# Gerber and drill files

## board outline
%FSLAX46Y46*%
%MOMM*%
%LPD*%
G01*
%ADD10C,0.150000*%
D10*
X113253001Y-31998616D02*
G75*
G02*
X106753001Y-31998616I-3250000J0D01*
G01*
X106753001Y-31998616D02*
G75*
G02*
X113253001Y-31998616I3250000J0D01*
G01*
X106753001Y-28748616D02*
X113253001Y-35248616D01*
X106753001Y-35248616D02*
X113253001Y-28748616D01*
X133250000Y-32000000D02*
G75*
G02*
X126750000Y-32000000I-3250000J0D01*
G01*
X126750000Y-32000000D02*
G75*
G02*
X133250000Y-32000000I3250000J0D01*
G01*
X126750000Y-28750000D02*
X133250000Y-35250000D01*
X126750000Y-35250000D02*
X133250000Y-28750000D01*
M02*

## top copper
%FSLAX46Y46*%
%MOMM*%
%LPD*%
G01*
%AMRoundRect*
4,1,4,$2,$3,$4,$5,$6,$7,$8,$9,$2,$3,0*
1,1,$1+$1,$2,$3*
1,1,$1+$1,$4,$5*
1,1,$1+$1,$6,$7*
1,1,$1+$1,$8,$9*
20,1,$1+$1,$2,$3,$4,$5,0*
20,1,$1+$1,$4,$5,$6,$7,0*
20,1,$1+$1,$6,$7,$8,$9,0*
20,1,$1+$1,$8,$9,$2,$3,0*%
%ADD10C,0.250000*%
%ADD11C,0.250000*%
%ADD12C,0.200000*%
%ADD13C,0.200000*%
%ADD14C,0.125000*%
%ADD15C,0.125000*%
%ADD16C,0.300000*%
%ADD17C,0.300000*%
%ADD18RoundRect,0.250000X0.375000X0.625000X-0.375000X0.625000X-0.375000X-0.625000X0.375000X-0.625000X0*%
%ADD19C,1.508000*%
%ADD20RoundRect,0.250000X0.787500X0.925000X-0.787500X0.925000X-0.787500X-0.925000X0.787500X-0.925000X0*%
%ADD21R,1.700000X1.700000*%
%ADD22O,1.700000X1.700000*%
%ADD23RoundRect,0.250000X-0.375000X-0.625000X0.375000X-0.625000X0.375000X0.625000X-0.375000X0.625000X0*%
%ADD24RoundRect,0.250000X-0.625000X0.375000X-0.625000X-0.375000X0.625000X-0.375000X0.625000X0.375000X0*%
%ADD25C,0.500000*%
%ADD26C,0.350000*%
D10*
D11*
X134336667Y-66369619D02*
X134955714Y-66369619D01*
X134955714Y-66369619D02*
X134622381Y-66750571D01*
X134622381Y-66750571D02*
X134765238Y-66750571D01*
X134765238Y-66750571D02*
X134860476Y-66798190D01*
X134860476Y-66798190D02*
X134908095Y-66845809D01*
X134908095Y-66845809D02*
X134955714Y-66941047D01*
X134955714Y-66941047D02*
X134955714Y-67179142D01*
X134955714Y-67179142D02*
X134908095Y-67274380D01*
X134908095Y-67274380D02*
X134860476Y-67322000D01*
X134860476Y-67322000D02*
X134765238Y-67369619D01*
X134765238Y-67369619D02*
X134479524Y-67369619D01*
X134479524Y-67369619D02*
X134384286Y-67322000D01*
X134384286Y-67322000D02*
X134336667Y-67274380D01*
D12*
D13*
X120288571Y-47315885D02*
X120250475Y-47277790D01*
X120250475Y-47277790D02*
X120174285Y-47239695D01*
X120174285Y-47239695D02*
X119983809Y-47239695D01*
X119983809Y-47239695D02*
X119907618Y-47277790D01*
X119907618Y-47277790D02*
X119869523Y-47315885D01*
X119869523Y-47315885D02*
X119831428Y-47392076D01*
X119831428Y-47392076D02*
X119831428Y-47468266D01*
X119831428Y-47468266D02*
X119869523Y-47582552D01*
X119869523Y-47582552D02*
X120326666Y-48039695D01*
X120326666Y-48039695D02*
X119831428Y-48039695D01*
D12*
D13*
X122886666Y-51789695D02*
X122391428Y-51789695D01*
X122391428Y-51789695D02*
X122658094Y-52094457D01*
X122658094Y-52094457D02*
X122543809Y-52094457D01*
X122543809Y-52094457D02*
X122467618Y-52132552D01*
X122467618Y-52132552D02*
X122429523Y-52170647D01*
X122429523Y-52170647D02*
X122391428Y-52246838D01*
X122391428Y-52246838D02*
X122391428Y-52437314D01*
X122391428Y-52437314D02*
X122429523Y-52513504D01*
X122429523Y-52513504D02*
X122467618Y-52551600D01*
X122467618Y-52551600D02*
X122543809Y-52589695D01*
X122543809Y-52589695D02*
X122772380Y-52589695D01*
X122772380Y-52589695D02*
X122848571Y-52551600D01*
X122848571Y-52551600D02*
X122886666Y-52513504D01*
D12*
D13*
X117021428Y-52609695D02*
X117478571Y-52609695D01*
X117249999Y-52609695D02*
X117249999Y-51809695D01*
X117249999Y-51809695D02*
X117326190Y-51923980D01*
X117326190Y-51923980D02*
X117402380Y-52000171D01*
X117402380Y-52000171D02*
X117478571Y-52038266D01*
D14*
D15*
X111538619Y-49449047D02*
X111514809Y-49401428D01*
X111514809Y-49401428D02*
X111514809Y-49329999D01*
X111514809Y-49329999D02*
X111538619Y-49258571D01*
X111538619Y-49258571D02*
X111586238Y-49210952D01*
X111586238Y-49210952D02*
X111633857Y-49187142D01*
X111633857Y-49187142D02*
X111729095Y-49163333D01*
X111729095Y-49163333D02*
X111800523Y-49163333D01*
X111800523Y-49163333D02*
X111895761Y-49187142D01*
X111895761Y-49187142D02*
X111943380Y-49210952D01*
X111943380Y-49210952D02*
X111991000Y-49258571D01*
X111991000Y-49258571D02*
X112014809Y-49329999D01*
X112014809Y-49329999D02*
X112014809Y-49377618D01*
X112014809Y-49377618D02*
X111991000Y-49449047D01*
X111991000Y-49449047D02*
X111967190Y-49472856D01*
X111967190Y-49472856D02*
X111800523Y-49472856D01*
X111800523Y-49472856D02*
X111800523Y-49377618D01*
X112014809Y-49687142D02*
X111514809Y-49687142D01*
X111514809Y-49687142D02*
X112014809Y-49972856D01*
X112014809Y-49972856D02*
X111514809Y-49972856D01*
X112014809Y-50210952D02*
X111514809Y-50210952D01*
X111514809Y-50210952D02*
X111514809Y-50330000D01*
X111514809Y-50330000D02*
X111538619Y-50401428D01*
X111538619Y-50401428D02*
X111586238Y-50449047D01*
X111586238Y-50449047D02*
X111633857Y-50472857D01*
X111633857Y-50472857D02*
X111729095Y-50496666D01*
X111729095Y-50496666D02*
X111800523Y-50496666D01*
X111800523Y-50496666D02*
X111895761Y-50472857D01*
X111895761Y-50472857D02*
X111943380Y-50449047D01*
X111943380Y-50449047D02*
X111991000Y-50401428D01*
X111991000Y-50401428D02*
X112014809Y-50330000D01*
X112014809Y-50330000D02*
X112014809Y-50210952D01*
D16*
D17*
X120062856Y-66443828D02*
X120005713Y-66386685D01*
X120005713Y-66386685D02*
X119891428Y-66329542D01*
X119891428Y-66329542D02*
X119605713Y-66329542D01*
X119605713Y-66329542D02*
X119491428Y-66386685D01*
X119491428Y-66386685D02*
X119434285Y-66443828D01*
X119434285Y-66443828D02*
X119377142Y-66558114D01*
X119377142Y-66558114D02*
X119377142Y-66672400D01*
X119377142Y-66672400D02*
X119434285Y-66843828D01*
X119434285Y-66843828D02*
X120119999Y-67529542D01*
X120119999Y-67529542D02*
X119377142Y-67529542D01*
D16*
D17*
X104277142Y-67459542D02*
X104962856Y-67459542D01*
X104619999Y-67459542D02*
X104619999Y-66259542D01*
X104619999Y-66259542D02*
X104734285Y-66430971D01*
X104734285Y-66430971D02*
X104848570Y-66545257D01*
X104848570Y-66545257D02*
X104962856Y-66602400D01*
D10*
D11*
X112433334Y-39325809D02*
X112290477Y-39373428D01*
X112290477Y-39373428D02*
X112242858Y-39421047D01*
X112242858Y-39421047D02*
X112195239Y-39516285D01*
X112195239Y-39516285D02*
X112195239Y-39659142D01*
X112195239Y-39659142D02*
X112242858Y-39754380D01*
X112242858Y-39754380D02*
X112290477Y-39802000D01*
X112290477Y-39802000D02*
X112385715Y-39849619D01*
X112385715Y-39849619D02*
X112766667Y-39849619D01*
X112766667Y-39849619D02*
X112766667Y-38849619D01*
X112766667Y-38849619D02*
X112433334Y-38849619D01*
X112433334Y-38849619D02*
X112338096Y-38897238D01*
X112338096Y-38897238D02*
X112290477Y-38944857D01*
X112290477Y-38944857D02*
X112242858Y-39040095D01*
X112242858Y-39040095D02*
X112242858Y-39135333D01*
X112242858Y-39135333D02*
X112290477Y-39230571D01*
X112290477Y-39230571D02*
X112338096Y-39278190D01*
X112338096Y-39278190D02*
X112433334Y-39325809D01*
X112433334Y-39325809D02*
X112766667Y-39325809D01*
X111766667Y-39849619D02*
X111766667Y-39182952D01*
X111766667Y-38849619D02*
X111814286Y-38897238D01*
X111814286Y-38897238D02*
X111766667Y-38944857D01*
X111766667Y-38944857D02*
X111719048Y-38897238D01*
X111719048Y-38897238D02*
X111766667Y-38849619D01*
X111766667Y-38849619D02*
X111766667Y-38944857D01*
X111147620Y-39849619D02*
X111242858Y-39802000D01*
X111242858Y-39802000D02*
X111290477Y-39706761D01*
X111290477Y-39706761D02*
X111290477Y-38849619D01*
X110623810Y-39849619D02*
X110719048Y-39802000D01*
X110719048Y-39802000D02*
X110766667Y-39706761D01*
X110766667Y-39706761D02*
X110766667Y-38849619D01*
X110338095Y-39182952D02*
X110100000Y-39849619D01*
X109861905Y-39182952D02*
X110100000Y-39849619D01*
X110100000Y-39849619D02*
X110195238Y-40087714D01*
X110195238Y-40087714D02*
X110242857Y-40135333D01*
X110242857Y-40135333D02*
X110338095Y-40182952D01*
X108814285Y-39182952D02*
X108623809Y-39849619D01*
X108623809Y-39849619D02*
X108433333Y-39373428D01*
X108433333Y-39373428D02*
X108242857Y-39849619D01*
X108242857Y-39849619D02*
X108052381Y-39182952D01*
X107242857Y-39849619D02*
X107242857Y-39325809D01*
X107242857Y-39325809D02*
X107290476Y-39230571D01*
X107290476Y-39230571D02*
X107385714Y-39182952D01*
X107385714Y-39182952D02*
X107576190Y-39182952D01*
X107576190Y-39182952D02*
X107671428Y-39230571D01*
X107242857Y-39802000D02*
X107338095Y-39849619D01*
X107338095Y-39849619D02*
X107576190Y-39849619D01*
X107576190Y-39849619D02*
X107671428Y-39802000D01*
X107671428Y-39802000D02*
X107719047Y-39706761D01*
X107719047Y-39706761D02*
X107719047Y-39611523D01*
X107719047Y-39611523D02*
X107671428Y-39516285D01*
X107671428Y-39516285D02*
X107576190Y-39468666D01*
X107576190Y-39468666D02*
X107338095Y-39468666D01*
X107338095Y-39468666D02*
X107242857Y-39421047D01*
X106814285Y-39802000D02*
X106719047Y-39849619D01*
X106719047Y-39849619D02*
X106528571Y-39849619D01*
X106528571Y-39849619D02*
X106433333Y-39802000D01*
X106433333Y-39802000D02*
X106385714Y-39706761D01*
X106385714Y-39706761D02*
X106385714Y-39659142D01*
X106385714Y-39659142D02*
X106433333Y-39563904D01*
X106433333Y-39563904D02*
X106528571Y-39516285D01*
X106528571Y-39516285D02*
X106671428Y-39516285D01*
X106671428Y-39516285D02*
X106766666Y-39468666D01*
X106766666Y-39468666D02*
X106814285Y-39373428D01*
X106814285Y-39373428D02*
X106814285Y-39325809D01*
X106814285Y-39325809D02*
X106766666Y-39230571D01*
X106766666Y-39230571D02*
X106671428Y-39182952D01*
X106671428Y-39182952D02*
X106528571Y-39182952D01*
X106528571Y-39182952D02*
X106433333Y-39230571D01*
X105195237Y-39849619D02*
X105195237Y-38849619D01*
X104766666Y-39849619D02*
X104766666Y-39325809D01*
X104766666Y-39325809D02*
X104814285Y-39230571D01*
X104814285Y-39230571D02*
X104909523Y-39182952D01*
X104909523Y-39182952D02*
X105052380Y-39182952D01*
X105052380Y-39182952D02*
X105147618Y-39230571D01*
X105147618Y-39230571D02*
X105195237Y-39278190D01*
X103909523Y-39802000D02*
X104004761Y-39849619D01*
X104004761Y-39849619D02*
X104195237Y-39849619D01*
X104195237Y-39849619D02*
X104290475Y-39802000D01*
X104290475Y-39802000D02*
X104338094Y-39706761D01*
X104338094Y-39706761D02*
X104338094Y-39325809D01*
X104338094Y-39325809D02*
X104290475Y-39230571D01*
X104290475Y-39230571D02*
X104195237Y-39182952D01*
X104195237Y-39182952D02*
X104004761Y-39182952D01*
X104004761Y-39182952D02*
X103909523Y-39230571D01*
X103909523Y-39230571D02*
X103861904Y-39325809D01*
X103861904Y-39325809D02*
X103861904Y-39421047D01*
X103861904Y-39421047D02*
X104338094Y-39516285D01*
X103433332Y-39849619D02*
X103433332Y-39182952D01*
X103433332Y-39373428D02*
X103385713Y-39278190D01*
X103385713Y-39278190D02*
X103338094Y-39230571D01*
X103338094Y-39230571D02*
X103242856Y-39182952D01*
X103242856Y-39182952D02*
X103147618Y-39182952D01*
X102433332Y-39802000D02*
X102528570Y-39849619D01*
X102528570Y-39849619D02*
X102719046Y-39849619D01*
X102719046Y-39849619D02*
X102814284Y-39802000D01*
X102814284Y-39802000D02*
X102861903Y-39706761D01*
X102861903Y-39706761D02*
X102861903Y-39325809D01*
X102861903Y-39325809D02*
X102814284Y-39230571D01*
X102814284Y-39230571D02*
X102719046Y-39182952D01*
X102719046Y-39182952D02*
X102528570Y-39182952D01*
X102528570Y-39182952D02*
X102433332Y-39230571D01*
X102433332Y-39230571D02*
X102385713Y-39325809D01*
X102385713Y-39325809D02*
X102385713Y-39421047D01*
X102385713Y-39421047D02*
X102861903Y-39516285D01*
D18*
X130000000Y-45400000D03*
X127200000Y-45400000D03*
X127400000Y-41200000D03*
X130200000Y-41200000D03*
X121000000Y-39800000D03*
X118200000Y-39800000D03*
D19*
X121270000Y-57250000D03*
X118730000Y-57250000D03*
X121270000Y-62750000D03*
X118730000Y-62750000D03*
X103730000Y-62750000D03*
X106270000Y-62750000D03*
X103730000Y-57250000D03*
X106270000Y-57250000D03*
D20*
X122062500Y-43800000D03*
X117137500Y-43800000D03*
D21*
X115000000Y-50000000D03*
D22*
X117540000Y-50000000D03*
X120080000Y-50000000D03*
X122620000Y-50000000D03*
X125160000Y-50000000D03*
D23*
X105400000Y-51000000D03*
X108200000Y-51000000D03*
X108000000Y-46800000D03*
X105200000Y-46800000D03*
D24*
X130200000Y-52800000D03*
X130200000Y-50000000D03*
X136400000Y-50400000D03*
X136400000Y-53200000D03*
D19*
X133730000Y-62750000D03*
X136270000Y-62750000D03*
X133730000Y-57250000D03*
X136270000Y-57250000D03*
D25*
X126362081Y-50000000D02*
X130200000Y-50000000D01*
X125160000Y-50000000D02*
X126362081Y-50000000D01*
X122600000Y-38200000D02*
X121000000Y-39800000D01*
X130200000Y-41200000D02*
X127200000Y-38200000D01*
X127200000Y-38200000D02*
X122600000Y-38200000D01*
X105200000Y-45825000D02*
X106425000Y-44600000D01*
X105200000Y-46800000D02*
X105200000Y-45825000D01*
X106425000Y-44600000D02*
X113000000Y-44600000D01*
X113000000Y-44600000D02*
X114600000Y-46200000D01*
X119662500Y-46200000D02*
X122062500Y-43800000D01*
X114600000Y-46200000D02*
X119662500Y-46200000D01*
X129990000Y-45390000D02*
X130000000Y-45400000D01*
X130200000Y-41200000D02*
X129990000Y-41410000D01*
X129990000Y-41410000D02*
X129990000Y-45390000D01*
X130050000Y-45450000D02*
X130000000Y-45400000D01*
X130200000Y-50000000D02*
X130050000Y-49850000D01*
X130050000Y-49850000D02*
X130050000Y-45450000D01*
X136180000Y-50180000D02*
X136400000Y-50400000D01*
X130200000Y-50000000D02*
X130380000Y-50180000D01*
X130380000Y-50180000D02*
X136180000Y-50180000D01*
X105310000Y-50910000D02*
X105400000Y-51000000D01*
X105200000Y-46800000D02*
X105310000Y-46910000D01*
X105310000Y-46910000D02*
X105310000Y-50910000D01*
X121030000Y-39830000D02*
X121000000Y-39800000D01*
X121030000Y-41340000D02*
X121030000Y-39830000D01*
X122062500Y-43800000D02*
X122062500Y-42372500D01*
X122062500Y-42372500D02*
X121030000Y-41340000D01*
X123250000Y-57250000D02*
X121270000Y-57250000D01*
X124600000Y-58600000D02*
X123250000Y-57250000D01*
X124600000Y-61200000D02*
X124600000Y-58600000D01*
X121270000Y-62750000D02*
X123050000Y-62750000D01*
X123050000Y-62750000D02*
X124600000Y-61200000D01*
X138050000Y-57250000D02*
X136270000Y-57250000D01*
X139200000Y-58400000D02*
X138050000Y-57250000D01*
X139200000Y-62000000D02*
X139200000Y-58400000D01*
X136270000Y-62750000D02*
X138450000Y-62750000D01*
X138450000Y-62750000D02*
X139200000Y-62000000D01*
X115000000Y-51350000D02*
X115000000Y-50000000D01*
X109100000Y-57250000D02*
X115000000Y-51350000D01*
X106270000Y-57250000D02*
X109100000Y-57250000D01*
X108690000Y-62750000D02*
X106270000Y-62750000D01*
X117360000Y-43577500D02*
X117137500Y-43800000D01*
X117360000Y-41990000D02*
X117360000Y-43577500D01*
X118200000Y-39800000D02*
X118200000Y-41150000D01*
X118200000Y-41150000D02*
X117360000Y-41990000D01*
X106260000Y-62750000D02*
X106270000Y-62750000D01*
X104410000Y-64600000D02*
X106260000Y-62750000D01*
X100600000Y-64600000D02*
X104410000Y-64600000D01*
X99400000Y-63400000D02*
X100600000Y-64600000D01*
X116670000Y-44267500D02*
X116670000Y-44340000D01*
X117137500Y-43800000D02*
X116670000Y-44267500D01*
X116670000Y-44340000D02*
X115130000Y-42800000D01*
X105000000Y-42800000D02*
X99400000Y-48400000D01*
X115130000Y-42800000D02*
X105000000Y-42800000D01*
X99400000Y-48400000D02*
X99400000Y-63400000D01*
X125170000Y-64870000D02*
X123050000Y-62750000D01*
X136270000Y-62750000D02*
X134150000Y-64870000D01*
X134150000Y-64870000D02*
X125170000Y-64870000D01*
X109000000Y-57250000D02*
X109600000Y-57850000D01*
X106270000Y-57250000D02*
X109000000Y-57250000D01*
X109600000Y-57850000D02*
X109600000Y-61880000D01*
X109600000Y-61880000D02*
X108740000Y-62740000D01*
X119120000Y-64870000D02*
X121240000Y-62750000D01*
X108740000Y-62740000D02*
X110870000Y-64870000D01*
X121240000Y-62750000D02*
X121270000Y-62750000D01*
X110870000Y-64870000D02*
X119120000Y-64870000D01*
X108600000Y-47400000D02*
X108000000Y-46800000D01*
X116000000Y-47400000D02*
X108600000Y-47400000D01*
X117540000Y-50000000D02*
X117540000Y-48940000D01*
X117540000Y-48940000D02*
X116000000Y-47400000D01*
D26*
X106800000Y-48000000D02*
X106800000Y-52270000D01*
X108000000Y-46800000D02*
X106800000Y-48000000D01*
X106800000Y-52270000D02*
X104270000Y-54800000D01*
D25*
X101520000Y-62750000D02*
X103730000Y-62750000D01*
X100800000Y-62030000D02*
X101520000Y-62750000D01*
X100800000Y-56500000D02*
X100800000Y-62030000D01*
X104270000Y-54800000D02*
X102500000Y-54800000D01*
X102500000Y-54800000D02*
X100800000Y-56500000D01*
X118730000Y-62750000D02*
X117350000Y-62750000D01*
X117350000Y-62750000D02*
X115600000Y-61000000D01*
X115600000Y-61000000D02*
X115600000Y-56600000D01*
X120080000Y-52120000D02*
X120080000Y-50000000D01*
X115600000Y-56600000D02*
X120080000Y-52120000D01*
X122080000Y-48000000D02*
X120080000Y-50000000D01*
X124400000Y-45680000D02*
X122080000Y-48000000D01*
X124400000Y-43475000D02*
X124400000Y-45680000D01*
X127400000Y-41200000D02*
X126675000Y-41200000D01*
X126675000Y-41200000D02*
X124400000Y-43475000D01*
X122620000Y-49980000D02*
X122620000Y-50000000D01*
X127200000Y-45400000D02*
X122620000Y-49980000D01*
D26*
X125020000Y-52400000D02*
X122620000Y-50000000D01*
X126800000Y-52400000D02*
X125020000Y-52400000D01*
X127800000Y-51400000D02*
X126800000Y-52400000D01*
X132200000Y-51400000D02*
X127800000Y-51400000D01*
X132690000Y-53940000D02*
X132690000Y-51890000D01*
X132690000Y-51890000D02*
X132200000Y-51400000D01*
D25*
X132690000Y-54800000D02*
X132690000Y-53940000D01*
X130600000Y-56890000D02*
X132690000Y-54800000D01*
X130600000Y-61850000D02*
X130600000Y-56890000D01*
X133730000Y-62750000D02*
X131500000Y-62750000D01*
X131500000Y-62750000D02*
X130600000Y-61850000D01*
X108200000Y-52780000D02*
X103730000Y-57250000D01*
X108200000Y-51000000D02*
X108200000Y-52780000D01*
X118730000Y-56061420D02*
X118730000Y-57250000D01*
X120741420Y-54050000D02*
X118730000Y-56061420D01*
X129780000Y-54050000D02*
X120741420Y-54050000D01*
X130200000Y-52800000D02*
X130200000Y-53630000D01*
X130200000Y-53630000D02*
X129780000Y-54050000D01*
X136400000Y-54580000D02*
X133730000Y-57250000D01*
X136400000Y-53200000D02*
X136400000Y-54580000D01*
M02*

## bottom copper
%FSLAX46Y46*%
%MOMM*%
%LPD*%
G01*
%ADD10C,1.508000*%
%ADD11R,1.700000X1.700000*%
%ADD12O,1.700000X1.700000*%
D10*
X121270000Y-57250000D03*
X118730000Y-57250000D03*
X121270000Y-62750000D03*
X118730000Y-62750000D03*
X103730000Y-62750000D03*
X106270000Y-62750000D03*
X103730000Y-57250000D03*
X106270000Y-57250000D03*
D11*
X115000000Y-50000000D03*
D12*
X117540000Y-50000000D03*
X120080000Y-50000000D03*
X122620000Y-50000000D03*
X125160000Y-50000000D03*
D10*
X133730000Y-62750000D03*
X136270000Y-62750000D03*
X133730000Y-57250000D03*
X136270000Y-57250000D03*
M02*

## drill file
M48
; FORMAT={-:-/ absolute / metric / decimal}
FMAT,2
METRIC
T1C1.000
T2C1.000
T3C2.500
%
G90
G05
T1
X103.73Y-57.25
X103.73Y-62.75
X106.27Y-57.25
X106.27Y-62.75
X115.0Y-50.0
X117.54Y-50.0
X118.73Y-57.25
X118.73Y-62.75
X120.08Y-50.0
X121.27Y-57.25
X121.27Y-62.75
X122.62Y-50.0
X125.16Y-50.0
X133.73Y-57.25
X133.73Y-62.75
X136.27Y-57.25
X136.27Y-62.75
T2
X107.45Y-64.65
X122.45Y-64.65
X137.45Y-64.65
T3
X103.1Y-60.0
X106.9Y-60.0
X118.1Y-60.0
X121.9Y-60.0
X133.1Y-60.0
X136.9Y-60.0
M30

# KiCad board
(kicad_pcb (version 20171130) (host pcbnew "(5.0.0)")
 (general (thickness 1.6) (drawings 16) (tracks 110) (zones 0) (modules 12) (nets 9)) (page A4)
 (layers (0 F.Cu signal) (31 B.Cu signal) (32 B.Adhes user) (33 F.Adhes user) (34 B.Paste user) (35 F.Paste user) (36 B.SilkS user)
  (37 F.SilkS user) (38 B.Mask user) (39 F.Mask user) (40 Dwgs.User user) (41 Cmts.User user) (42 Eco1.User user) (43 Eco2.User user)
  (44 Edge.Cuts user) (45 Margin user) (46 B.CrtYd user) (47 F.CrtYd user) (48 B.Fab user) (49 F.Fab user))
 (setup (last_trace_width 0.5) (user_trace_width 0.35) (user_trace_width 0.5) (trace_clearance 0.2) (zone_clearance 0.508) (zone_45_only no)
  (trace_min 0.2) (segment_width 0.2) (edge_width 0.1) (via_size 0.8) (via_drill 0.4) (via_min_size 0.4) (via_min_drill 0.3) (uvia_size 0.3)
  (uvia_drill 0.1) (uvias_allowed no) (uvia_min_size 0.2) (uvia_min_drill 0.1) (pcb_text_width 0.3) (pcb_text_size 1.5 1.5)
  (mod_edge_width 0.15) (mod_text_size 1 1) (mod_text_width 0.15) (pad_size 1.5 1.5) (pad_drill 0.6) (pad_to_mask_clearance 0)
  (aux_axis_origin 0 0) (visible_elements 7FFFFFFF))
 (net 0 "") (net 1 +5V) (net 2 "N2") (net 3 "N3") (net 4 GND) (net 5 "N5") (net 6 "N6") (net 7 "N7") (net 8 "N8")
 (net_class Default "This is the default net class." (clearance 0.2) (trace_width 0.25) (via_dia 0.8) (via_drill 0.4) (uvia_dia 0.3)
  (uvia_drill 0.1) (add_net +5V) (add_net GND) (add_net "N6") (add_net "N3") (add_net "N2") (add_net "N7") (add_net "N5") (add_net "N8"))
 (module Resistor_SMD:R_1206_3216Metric (layer F.Cu) (at 128.6 45.4 180)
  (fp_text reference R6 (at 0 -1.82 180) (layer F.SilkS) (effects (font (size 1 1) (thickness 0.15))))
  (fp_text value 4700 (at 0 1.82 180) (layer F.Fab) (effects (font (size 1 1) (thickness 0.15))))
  (pad 1 smd roundrect (at -1.4 0 180) (size 1.25 1.75) (layers F.Cu F.Paste F.Mask) (roundrect_rratio 0.2) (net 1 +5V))
  (pad 2 smd roundrect (at 1.4 0 180) (size 1.25 1.75) (layers F.Cu F.Paste F.Mask) (roundrect_rratio 0.2) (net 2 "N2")))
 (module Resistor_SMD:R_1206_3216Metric (layer F.Cu) (at 128.8 41.2 180)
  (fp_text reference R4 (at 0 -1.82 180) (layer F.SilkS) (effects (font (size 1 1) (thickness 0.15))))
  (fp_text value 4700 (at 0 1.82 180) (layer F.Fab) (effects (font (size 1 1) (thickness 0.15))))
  (pad 2 smd roundrect (at 1.4 0 180) (size 1.25 1.75) (layers F.Cu F.Paste F.Mask) (roundrect_rratio 0.2) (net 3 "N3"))
  (pad 1 smd roundrect (at -1.4 0 180) (size 1.25 1.75) (layers F.Cu F.Paste F.Mask) (roundrect_rratio 0.2) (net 1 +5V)))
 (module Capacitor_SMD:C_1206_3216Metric (layer F.Cu) (at 119.6 39.8 180)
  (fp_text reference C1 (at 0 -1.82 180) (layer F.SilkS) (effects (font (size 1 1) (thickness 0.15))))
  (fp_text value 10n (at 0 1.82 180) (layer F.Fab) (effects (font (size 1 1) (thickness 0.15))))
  (pad 1 smd roundrect (at -1.4 0 180) (size 1.25 1.75) (layers F.Cu F.Paste F.Mask) (roundrect_rratio 0.2) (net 1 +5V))
  (pad 2 smd roundrect (at 1.4 0 180) (size 1.25 1.75) (layers F.Cu F.Paste F.Mask) (roundrect_rratio 0.2) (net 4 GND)))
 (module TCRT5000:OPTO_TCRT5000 (layer F.Cu) (at 120 60 90)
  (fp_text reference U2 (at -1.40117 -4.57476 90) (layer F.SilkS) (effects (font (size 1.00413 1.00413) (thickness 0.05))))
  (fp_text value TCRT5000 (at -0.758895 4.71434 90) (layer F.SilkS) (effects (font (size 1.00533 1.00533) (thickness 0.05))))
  (pad Hole np_thru_hole circle (at 0 -1.9 90) (size 2.5 2.5) (drill 2.5) (layers *.Cu *.Mask F.SilkS))
  (pad Hole np_thru_hole circle (at 0 1.9 90) (size 2.5 2.5) (drill 2.5) (layers *.Cu *.Mask F.SilkS))
  (pad Hole np_thru_hole circle (at -4.65 2.45 90) (size 1 1) (drill 1) (layers *.Cu *.Mask F.SilkS))
  (pad CATH thru_hole circle (at 2.75 1.27 90) (size 1.508 1.508) (drill 1) (layers *.Cu *.Mask) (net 4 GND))
  (pad A thru_hole circle (at 2.75 -1.27 90) (size 1.508 1.508) (drill 1) (layers *.Cu *.Mask) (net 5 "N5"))
  (pad E thru_hole circle (at -2.75 1.27 90) (size 1.508 1.508) (drill 1) (layers *.Cu *.Mask) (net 4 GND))
  (pad COLL thru_hole circle (at -2.75 -1.27 90) (size 1.508 1.508) (drill 1) (layers *.Cu *.Mask) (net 3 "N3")))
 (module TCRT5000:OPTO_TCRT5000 (layer F.Cu) (at 105 60 90)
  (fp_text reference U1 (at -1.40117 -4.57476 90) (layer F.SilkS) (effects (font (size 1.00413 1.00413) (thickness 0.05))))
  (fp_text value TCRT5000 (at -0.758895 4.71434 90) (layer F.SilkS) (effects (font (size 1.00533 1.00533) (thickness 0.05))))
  (pad COLL thru_hole circle (at -2.75 -1.27 90) (size 1.508 1.508) (drill 1) (layers *.Cu *.Mask) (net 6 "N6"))
  (pad E thru_hole circle (at -2.75 1.27 90) (size 1.508 1.508) (drill 1) (layers *.Cu *.Mask) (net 4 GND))
  (pad A thru_hole circle (at 2.75 -1.27 90) (size 1.508 1.508) (drill 1) (layers *.Cu *.Mask) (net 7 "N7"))
  (pad CATH thru_hole circle (at 2.75 1.27 90) (size 1.508 1.508) (drill 1) (layers *.Cu *.Mask) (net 4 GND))
  (pad Hole np_thru_hole circle (at -4.65 2.45 90) (size 1 1) (drill 1) (layers *.Cu *.Mask F.SilkS))
  (pad Hole np_thru_hole circle (at 0 1.9 90) (size 2.5 2.5) (drill 2.5) (layers *.Cu *.Mask F.SilkS))
  (pad Hole np_thru_hole circle (at 0 -1.9 90) (size 2.5 2.5) (drill 2.5) (layers *.Cu *.Mask F.SilkS)))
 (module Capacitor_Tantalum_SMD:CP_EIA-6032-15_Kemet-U (layer F.Cu) (at 119.6 43.8 180)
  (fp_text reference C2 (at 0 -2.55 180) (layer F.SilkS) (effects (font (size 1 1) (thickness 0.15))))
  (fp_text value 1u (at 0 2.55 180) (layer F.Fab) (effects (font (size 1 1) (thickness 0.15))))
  (pad 1 smd roundrect (at -2.4625 0 180) (size 2.075 2.35) (layers F.Cu F.Paste F.Mask) (roundrect_rratio 0.120482) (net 1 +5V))
  (pad 2 smd roundrect (at 2.4625 0 180) (size 2.075 2.35) (layers F.Cu F.Paste F.Mask) (roundrect_rratio 0.120482) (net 4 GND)))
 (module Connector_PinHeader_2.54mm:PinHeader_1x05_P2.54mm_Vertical (layer F.Cu) (at 115 50 90)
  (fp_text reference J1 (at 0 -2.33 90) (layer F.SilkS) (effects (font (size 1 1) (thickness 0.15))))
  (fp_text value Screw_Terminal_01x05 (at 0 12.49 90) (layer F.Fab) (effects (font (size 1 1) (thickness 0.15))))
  (pad 1 thru_hole rect (at 0 0 90) (size 1.7 1.7) (drill 1) (layers *.Cu *.Mask) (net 4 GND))
  (pad 2 thru_hole oval (at 0 2.54 90) (size 1.7 1.7) (drill 1) (layers *.Cu *.Mask) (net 6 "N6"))
  (pad 3 thru_hole oval (at 0 5.08 90) (size 1.7 1.7) (drill 1) (layers *.Cu *.Mask) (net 3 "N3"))
  (pad 4 thru_hole oval (at 0 7.62 90) (size 1.7 1.7) (drill 1) (layers *.Cu *.Mask) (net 2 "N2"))
  (pad 5 thru_hole oval (at 0 10.16 90) (size 1.7 1.7) (drill 1) (layers *.Cu *.Mask) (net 1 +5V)))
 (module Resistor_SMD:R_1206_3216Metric (layer F.Cu) (at 106.8 51)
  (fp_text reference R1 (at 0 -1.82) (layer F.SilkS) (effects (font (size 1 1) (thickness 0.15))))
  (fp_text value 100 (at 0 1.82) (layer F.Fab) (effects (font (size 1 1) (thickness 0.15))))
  (pad 1 smd roundrect (at -1.4 0) (size 1.25 1.75) (layers F.Cu F.Paste F.Mask) (roundrect_rratio 0.2) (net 1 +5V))
  (pad 2 smd roundrect (at 1.4 0) (size 1.25 1.75) (layers F.Cu F.Paste F.Mask) (roundrect_rratio 0.2) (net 7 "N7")))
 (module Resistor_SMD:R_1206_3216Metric (layer F.Cu) (at 106.6 46.8)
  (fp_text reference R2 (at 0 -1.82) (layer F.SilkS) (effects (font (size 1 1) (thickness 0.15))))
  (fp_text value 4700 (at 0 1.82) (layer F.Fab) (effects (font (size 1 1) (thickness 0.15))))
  (pad 2 smd roundrect (at 1.4 0) (size 1.25 1.75) (layers F.Cu F.Paste F.Mask) (roundrect_rratio 0.2) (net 6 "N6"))
  (pad 1 smd roundrect (at -1.4 0) (size 1.25 1.75) (layers F.Cu F.Paste F.Mask) (roundrect_rratio 0.2) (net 1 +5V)))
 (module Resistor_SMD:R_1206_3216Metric (layer F.Cu) (at 130.2 51.4 270)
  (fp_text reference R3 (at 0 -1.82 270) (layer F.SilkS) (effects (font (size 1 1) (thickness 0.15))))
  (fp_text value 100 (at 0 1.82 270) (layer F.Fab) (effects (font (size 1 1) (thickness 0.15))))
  (pad 2 smd roundrect (at 1.4 0 270) (size 1.25 1.75) (layers F.Cu F.Paste F.Mask) (roundrect_rratio 0.2) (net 5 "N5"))
  (pad 1 smd roundrect (at -1.4 0 270) (size 1.25 1.75) (layers F.Cu F.Paste F.Mask) (roundrect_rratio 0.2) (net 1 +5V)))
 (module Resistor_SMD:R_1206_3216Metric (layer F.Cu) (at 136.4 51.8 270)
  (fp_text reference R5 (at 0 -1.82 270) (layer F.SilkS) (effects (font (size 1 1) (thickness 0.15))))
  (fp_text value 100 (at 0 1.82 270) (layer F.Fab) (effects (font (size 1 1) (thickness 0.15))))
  (pad 1 smd roundrect (at -1.4 0 270) (size 1.25 1.75) (layers F.Cu F.Paste F.Mask) (roundrect_rratio 0.2) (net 1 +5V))
  (pad 2 smd roundrect (at 1.4 0 270) (size 1.25 1.75) (layers F.Cu F.Paste F.Mask) (roundrect_rratio 0.2) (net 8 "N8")))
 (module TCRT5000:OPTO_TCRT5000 (layer F.Cu) (at 135 60 90)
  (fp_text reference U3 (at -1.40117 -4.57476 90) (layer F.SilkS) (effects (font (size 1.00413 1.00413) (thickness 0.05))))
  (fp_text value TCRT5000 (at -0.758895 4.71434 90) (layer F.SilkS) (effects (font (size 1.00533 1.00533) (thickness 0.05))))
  (pad COLL thru_hole circle (at -2.75 -1.27 90) (size 1.508 1.508) (drill 1) (layers *.Cu *.Mask) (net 2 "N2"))
  (pad E thru_hole circle (at -2.75 1.27 90) (size 1.508 1.508) (drill 1) (layers *.Cu *.Mask) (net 4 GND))
  (pad A thru_hole circle (at 2.75 -1.27 90) (size 1.508 1.508) (drill 1) (layers *.Cu *.Mask) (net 8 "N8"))
  (pad CATH thru_hole circle (at 2.75 1.27 90) (size 1.508 1.508) (drill 1) (layers *.Cu *.Mask) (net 4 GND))
  (pad Hole np_thru_hole circle (at -4.65 2.45 90) (size 1 1) (drill 1) (layers *.Cu *.Mask F.SilkS))
  (pad Hole np_thru_hole circle (at 0 1.9 90) (size 2.5 2.5) (drill 2.5) (layers *.Cu *.Mask F.SilkS))
  (pad Hole np_thru_hole circle (at 0 -1.9 90) (size 2.5 2.5) (drill 2.5) (layers *.Cu *.Mask F.SilkS)))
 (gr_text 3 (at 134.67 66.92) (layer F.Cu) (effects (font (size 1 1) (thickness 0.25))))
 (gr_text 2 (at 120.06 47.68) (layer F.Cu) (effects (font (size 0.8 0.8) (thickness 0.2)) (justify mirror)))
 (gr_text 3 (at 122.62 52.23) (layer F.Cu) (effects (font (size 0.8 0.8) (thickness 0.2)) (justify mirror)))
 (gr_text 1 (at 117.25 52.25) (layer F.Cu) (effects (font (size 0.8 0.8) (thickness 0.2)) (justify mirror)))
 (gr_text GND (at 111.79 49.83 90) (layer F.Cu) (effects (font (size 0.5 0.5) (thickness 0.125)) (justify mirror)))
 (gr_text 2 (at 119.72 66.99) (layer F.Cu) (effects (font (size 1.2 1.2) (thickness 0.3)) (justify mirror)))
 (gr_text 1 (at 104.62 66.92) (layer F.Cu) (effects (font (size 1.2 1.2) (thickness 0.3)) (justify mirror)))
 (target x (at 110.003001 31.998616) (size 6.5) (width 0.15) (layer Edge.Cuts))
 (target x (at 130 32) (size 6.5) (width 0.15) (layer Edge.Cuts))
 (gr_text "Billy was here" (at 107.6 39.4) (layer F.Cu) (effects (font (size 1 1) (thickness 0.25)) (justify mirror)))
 (segment (start 126.362081 50) (end 130.2 50) (width 0.5) (layer F.Cu) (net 1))
 (segment (start 125.16 50) (end 126.362081 50) (width 0.5) (layer F.Cu) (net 1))
 (segment (start 122.6 38.2) (end 121 39.8) (width 0.5) (layer F.Cu) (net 1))
 (segment (start 130.2 41.2) (end 127.2 38.2) (width 0.5) (layer F.Cu) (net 1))
 (segment (start 127.2 38.2) (end 122.6 38.2) (width 0.5) (layer F.Cu) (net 1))
 (segment (start 105.2 45.825) (end 106.425 44.6) (width 0.5) (layer F.Cu) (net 1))
 (segment (start 105.2 46.8) (end 105.2 45.825) (width 0.5) (layer F.Cu) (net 1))
 (segment (start 106.425 44.6) (end 113 44.6) (width 0.5) (layer F.Cu) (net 1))
 (segment (start 113 44.6) (end 114.6 46.2) (width 0.5) (layer F.Cu) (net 1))
 (segment (start 119.6625 46.2) (end 122.0625 43.8) (width 0.5) (layer F.Cu) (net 1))
 (segment (start 114.6 46.2) (end 119.6625 46.2) (width 0.5) (layer F.Cu) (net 1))
 (segment (start 129.99 45.39) (end 130 45.4) (width 0.5) (layer F.Cu) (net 1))
 (segment (start 130.2 41.2) (end 129.99 41.41) (width 0.5) (layer F.Cu) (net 1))
 (segment (start 129.99 41.41) (end 129.99 45.39) (width 0.5) (layer F.Cu) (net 1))
 (segment (start 130.05 45.45) (end 130 45.4) (width 0.5) (layer F.Cu) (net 1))
 (segment (start 130.2 50) (end 130.05 49.85) (width 0.5) (layer F.Cu) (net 1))
 (segment (start 130.05 49.85) (end 130.05 45.45) (width 0.5) (layer F.Cu) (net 1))
 (segment (start 136.18 50.18) (end 136.4 50.4) (width 0.5) (layer F.Cu) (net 1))
 (segment (start 130.2 50) (end 130.38 50.18) (width 0.5) (layer F.Cu) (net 1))
 (segment (start 130.38 50.18) (end 136.18 50.18) (width 0.5) (layer F.Cu) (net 1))
 (segment (start 105.31 50.91) (end 105.4 51) (width 0.5) (layer F.Cu) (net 1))
 (segment (start 105.2 46.8) (end 105.31 46.91) (width 0.5) (layer F.Cu) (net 1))
 (segment (start 105.31 46.91) (end 105.31 50.91) (width 0.5) (layer F.Cu) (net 1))
 (segment (start 121.03 39.83) (end 121 39.8) (width 0.5) (layer F.Cu) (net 1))
 (segment (start 121.03 41.34) (end 121.03 39.83) (width 0.5) (layer F.Cu) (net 1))
 (segment (start 122.0625 43.8) (end 122.0625 42.3725) (width 0.5) (layer F.Cu) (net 1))
 (segment (start 122.0625 42.3725) (end 121.03 41.34) (width 0.5) (layer F.Cu) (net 1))
 (segment (start 123.25 57.25) (end 121.27 57.25) (width 0.5) (layer F.Cu) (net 4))
 (segment (start 124.6 58.6) (end 123.25 57.25) (width 0.5) (layer F.Cu) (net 4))
 (segment (start 124.6 61.2) (end 124.6 58.6) (width 0.5) (layer F.Cu) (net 4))
 (segment (start 121.27 62.75) (end 123.05 62.75) (width 0.5) (layer F.Cu) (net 4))
 (segment (start 123.05 62.75) (end 124.6 61.2) (width 0.5) (layer F.Cu) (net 4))
 (segment (start 138.05 57.25) (end 136.27 57.25) (width 0.5) (layer F.Cu) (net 4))
 (segment (start 139.2 58.4) (end 138.05 57.25) (width 0.5) (layer F.Cu) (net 4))
 (segment (start 139.2 62) (end 139.2 58.4) (width 0.5) (layer F.Cu) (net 4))
 (segment (start 136.27 62.75) (end 138.45 62.75) (width 0.5) (layer F.Cu) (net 4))
 (segment (start 138.45 62.75) (end 139.2 62) (width 0.5) (layer F.Cu) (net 4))
 (segment (start 115 51.35) (end 115 50) (width 0.5) (layer F.Cu) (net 4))
 (segment (start 109.1 57.25) (end 115 51.35) (width 0.5) (layer F.Cu) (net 4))
 (segment (start 106.27 57.25) (end 109.1 57.25) (width 0.5) (layer F.Cu) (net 4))
 (segment (start 108.69 62.75) (end 106.27 62.75) (width 0.5) (layer F.Cu) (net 4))
 (segment (start 117.36 43.5775) (end 117.1375 43.8) (width 0.5) (layer F.Cu) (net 4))
 (segment (start 117.36 41.99) (end 117.36 43.5775) (width 0.5) (layer F.Cu) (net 4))
 (segment (start 118.2 39.8) (end 118.2 41.15) (width 0.5) (layer F.Cu) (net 4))
 (segment (start 118.2 41.15) (end 117.36 41.99) (width 0.5) (layer F.Cu) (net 4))
 (segment (start 106.26 62.75) (end 106.27 62.75) (width 0.5) (layer F.Cu) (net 4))
 (segment (start 104.41 64.6) (end 106.26 62.75) (width 0.5) (layer F.Cu) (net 4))
 (segment (start 100.6 64.6) (end 104.41 64.6) (width 0.5) (layer F.Cu) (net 4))
 (segment (start 99.4 63.4) (end 100.6 64.6) (width 0.5) (layer F.Cu) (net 4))
 (segment (start 116.67 44.2675) (end 116.67 44.34) (width 0.5) (layer F.Cu) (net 4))
 (segment (start 117.1375 43.8) (end 116.67 44.2675) (width 0.5) (layer F.Cu) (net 4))
 (segment (start 116.67 44.34) (end 115.13 42.8) (width 0.5) (layer F.Cu) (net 4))
 (segment (start 105 42.8) (end 99.4 48.4) (width 0.5) (layer F.Cu) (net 4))
 (segment (start 115.13 42.8) (end 105 42.8) (width 0.5) (layer F.Cu) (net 4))
 (segment (start 99.4 48.4) (end 99.4 63.4) (width 0.5) (layer F.Cu) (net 4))
 (segment (start 125.17 64.87) (end 123.05 62.75) (width 0.5) (layer F.Cu) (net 4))
 (segment (start 136.27 62.75) (end 134.15 64.87) (width 0.5) (layer F.Cu) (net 4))
 (segment (start 134.15 64.87) (end 125.17 64.87) (width 0.5) (layer F.Cu) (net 4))
 (segment (start 109 57.25) (end 109.6 57.85) (width 0.5) (layer F.Cu) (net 4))
 (segment (start 106.27 57.25) (end 109 57.25) (width 0.5) (layer F.Cu) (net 4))
 (segment (start 109.6 57.85) (end 109.6 61.88) (width 0.5) (layer F.Cu) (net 4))
 (segment (start 109.6 61.88) (end 108.74 62.74) (width 0.5) (layer F.Cu) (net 4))
 (segment (start 119.12 64.87) (end 121.24 62.75) (width 0.5) (layer F.Cu) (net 4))
 (segment (start 108.74 62.74) (end 110.87 64.87) (width 0.5) (layer F.Cu) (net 4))
 (segment (start 121.24 62.75) (end 121.27 62.75) (width 0.5) (layer F.Cu) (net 4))
 (segment (start 110.87 64.87) (end 119.12 64.87) (width 0.5) (layer F.Cu) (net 4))
 (segment (start 108.6 47.4) (end 108 46.8) (width 0.5) (layer F.Cu) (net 6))
 (segment (start 116 47.4) (end 108.6 47.4) (width 0.5) (layer F.Cu) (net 6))
 (segment (start 117.54 50) (end 117.54 48.94) (width 0.5) (layer F.Cu) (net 6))
 (segment (start 117.54 48.94) (end 116 47.4) (width 0.5) (layer F.Cu) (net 6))
 (segment (start 106.8 48) (end 106.8 52.27) (width 0.35) (layer F.Cu) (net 6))
 (segment (start 108 46.8) (end 106.8 48) (width 0.35) (layer F.Cu) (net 6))
 (segment (start 106.8 52.27) (end 104.27 54.8) (width 0.35) (layer F.Cu) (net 6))
 (segment (start 101.52 62.75) (end 103.73 62.75) (width 0.5) (layer F.Cu) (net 6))
 (segment (start 100.8 62.03) (end 101.52 62.75) (width 0.5) (layer F.Cu) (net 6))
 (segment (start 100.8 56.5) (end 100.8 62.03) (width 0.5) (layer F.Cu) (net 6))
 (segment (start 104.27 54.8) (end 102.5 54.8) (width 0.5) (layer F.Cu) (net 6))
 (segment (start 102.5 54.8) (end 100.8 56.5) (width 0.5) (layer F.Cu) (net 6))
 (segment (start 118.73 62.75) (end 117.35 62.75) (width 0.5) (layer F.Cu) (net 3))
 (segment (start 117.35 62.75) (end 115.6 61) (width 0.5) (layer F.Cu) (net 3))
 (segment (start 115.6 61) (end 115.6 56.6) (width 0.5) (layer F.Cu) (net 3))
 (segment (start 120.08 52.12) (end 120.08 50) (width 0.5) (layer F.Cu) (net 3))
 (segment (start 115.6 56.6) (end 120.08 52.12) (width 0.5) (layer F.Cu) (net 3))
 (segment (start 122.08 48) (end 120.08 50) (width 0.5) (layer F.Cu) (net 3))
 (segment (start 124.4 45.68) (end 122.08 48) (width 0.5) (layer F.Cu) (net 3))
 (segment (start 124.4 43.475) (end 124.4 45.68) (width 0.5) (layer F.Cu) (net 3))
 (segment (start 127.4 41.2) (end 126.675 41.2) (width 0.5) (layer F.Cu) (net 3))
 (segment (start 126.675 41.2) (end 124.4 43.475) (width 0.5) (layer F.Cu) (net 3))
 (segment (start 122.62 49.98) (end 122.62 50) (width 0.5) (layer F.Cu) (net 2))
 (segment (start 127.2 45.4) (end 122.62 49.98) (width 0.5) (layer F.Cu) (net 2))
 (segment (start 125.02 52.4) (end 122.62 50) (width 0.35) (layer F.Cu) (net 2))
 (segment (start 126.8 52.4) (end 125.02 52.4) (width 0.35) (layer F.Cu) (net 2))
 (segment (start 127.8 51.4) (end 126.8 52.4) (width 0.35) (layer F.Cu) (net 2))
 (segment (start 132.2 51.4) (end 127.8 51.4) (width 0.35) (layer F.Cu) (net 2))
 (segment (start 132.69 53.94) (end 132.69 51.89) (width 0.35) (layer F.Cu) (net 2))
 (segment (start 132.69 51.89) (end 132.2 51.4) (width 0.35) (layer F.Cu) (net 2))
 (segment (start 132.69 54.8) (end 132.69 53.94) (width 0.5) (layer F.Cu) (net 2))
 (segment (start 130.6 56.89) (end 132.69 54.8) (width 0.5) (layer F.Cu) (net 2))
 (segment (start 130.6 61.85) (end 130.6 56.89) (width 0.5) (layer F.Cu) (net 2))
 (segment (start 133.73 62.75) (end 131.5 62.75) (width 0.5) (layer F.Cu) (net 2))
 (segment (start 131.5 62.75) (end 130.6 61.85) (width 0.5) (layer F.Cu) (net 2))
 (segment (start 108.2 52.78) (end 103.73 57.25) (width 0.5) (layer F.Cu) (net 7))
 (segment (start 108.2 51) (end 108.2 52.78) (width 0.5) (layer F.Cu) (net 7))
 (segment (start 118.73 56.06142) (end 118.73 57.25) (width 0.5) (layer F.Cu) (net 5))
 (segment (start 120.74142 54.05) (end 118.73 56.06142) (width 0.5) (layer F.Cu) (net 5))
 (segment (start 129.78 54.05) (end 120.74142 54.05) (width 0.5) (layer F.Cu) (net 5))
 (segment (start 130.2 52.8) (end 130.2 53.63) (width 0.5) (layer F.Cu) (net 5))
 (segment (start 130.2 53.63) (end 129.78 54.05) (width 0.5) (layer F.Cu) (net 5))
 (segment (start 136.4 54.58) (end 133.73 57.25) (width 0.5) (layer F.Cu) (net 8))
 (segment (start 136.4 53.2) (end 136.4 54.58) (width 0.5) (layer F.Cu) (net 8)))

